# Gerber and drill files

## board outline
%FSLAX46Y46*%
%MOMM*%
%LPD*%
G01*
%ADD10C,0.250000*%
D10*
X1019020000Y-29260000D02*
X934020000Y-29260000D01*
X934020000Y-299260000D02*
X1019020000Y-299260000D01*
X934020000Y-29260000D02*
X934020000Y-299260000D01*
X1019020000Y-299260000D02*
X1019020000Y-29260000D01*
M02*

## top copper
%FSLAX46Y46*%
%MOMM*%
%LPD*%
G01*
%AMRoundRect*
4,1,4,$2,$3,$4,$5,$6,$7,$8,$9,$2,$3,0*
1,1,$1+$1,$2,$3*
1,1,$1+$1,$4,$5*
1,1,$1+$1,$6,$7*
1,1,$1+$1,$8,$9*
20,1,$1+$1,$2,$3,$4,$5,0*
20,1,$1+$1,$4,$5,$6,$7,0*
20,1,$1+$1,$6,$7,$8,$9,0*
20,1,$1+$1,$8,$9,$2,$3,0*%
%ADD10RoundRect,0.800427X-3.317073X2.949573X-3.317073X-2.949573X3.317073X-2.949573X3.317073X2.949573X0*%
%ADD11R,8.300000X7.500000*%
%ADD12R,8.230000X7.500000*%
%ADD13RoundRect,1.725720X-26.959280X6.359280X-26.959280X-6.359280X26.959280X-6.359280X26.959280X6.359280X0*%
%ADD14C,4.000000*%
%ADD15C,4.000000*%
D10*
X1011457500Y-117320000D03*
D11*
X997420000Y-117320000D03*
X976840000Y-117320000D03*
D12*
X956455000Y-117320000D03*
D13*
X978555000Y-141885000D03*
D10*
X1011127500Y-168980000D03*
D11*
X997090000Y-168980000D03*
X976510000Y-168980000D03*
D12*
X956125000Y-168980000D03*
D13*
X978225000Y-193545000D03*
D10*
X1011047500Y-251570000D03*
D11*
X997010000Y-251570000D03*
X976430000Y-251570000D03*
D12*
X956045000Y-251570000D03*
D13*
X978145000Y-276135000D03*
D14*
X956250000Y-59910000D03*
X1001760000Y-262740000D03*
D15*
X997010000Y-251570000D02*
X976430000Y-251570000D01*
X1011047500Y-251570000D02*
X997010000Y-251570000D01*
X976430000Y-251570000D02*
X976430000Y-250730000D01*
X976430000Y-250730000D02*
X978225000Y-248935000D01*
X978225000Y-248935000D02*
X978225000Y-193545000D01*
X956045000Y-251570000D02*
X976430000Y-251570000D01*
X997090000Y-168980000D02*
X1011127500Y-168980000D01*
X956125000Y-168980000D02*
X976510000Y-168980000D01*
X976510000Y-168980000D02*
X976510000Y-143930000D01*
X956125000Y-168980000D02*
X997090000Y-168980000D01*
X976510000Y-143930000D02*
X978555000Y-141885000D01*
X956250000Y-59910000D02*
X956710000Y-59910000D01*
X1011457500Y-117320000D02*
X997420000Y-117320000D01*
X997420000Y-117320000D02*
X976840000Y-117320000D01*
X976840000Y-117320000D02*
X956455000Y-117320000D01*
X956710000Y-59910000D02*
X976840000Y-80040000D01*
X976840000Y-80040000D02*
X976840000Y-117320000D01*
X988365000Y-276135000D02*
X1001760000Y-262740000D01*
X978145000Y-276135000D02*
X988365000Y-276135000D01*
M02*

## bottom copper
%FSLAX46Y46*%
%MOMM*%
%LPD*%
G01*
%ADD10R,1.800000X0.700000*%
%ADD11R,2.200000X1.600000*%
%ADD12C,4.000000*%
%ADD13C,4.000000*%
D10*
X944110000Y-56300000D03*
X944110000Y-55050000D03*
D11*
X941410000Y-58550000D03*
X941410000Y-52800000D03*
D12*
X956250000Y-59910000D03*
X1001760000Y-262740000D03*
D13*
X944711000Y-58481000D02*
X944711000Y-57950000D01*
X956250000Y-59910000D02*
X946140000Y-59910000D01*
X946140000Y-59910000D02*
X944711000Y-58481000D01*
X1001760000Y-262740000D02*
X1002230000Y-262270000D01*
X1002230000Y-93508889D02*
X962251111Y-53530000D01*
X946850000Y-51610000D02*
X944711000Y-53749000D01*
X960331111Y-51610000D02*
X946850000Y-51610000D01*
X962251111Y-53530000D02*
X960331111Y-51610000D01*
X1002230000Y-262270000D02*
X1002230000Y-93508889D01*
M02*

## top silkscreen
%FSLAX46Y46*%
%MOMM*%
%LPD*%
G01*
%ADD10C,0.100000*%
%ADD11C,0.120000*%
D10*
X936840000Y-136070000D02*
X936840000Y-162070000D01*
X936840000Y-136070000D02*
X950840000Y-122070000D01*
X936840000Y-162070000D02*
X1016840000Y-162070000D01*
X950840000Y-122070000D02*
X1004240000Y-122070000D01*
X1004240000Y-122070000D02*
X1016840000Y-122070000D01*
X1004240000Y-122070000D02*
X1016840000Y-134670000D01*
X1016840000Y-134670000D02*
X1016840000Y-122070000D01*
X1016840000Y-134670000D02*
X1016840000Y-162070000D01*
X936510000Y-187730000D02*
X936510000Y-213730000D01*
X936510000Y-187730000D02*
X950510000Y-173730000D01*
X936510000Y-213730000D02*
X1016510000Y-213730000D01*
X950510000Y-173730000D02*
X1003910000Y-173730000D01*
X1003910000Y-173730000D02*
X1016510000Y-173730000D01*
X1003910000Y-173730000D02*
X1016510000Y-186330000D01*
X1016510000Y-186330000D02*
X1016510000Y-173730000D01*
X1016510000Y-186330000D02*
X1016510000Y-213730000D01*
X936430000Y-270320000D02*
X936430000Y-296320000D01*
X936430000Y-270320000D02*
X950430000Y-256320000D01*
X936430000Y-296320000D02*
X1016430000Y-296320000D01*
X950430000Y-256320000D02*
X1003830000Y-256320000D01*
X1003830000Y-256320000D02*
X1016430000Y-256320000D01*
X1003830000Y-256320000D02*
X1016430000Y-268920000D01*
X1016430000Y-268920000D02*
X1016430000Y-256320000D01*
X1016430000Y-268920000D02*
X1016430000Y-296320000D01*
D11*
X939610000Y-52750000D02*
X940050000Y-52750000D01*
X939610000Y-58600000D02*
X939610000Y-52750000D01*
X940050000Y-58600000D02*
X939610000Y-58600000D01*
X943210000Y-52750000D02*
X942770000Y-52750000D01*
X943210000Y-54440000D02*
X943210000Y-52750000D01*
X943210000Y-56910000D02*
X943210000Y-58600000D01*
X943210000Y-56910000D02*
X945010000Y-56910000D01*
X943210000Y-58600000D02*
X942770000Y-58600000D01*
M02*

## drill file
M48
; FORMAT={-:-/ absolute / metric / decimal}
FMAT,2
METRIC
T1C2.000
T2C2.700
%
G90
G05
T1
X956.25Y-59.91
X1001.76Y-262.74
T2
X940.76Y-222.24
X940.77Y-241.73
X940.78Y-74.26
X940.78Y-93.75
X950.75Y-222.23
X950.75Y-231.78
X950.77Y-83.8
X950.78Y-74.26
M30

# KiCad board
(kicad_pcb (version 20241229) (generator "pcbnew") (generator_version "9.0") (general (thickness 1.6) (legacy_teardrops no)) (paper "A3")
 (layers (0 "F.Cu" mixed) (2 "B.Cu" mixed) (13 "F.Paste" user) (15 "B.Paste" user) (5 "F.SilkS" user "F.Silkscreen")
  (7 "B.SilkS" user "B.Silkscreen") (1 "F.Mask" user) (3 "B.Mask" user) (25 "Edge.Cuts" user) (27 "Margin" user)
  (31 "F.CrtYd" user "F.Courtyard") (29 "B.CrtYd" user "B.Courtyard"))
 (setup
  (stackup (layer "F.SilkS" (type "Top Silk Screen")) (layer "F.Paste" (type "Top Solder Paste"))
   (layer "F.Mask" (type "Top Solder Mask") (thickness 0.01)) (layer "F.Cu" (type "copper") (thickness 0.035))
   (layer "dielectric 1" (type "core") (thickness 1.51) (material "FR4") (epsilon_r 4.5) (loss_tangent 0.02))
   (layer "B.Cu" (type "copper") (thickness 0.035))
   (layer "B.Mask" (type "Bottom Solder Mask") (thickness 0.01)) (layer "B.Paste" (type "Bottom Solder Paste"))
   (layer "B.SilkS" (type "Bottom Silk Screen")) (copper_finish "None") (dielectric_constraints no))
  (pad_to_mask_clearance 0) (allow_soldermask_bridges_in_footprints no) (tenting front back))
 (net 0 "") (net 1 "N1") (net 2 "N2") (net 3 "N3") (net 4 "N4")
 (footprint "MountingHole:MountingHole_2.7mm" (layer "F.Cu") (at 940.78 93.75)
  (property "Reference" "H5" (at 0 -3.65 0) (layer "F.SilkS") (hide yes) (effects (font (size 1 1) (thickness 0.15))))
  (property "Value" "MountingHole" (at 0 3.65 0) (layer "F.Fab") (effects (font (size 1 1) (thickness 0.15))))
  (pad "" np_thru_hole circle (at 0 0) (size 2.7 2.7) (drill 2.7) (layers "*.Cu" "*.Mask")))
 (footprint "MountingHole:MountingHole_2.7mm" (layer "F.Cu") (at 940.76 222.24)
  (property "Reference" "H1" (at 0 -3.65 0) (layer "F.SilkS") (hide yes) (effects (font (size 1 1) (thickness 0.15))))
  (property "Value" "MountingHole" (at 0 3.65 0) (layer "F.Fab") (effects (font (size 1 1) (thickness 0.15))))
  (pad "" np_thru_hole circle (at 0 0) (size 2.7 2.7) (drill 2.7) (layers "*.Cu" "*.Mask")))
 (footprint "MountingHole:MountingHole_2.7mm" (layer "F.Cu") (at 950.75 231.78)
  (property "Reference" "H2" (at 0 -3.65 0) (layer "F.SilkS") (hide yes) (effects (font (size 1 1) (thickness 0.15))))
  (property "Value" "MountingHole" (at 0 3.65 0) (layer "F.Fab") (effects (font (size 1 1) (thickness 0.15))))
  (pad "" np_thru_hole circle (at 0 0) (size 2.7 2.7) (drill 2.7) (layers "*.Cu" "*.Mask")))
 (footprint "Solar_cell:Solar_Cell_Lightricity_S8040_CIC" (layer "F.Cu") (at 936.84 122.07 -90)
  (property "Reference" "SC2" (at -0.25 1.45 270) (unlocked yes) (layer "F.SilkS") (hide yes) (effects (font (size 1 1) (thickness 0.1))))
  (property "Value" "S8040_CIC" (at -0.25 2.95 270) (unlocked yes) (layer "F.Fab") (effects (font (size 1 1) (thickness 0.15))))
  (fp_line (start 14 0) (end 40 0) (stroke (width 0.1) (type default)) (layer "F.SilkS"))
  (fp_line (start 14 0) (end 0 -14) (stroke (width 0.1) (type default)) (layer "F.SilkS"))
  (fp_line (start 40 0) (end 40 -80) (stroke (width 0.1) (type default)) (layer "F.SilkS"))
  (fp_line (start 0 -14) (end 0 -67.4) (stroke (width 0.1) (type default)) (layer "F.SilkS"))
  (fp_line (start 0 -67.4) (end 0 -80) (stroke (width 0.1) (type default)) (layer "F.SilkS"))
  (fp_line (start 0 -67.4) (end 12.6 -80) (stroke (width 0.1) (type default)) (layer "F.SilkS"))
  (fp_line (start 12.6 -80) (end 0 -80) (stroke (width 0.1) (type default)) (layer "F.SilkS"))
  (fp_line (start 12.6 -80) (end 40 -80) (stroke (width 0.1) (type default)) (layer "F.SilkS"))
  (pad "1" smd roundrect (at -4.75 -74.6175 270) (size 7.5 8.235) (layers "F.Cu" "F.Mask" "F.Paste") (roundrect_rratio 0.1067235859)
   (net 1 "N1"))
  (pad "1" smd rect (at -4.75 -60.58 270) (size 7.5 8.3) (layers "F.Cu" "F.Mask" "F.Paste") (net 1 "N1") (thermal_bridge_angle 45))
  (pad "1" smd rect (at -4.75 -40 270) (size 7.5 8.3) (layers "F.Cu" "F.Mask" "F.Paste") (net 1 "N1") (thermal_bridge_angle 45))
  (pad "1" smd rect (at -4.75 -19.615 270) (size 7.5 8.23) (layers "F.Cu" "F.Mask" "F.Paste") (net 1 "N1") (thermal_bridge_angle 45))
  (pad "2" smd roundrect (at 19.815 -41.715 270) (size 16.17 57.37) (layers "F.Cu" "F.Mask" "F.Paste") (roundrect_rratio 0.1067235859)
   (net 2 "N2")))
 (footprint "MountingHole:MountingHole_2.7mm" (layer "F.Cu") (at 940.77 241.73)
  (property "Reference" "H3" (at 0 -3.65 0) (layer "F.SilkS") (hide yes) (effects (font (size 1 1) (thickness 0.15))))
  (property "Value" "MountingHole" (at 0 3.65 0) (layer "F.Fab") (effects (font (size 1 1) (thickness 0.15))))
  (pad "" np_thru_hole circle (at 0 0) (size 2.7 2.7) (drill 2.7) (layers "*.Cu" "*.Mask")))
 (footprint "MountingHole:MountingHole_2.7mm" (layer "F.Cu") (at 950.77 83.8)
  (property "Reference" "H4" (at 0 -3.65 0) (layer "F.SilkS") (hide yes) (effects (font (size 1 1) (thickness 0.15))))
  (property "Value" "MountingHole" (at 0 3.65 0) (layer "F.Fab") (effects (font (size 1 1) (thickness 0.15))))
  (pad "" np_thru_hole circle (at 0 0) (size 2.7 2.7) (drill 2.7) (layers "*.Cu" "*.Mask")))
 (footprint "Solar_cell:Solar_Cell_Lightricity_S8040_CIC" (layer "F.Cu") (at 936.51 173.73 -90)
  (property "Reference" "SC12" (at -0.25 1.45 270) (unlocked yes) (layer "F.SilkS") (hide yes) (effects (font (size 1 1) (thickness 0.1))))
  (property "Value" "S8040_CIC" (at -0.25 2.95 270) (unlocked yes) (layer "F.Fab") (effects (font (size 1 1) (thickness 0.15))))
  (fp_line (start 14 0) (end 40 0) (stroke (width 0.1) (type default)) (layer "F.SilkS"))
  (fp_line (start 14 0) (end 0 -14) (stroke (width 0.1) (type default)) (layer "F.SilkS"))
  (fp_line (start 40 0) (end 40 -80) (stroke (width 0.1) (type default)) (layer "F.SilkS"))
  (fp_line (start 0 -14) (end 0 -67.4) (stroke (width 0.1) (type default)) (layer "F.SilkS"))
  (fp_line (start 0 -67.4) (end 0 -80) (stroke (width 0.1) (type default)) (layer "F.SilkS"))
  (fp_line (start 0 -67.4) (end 12.6 -80) (stroke (width 0.1) (type default)) (layer "F.SilkS"))
  (fp_line (start 12.6 -80) (end 0 -80) (stroke (width 0.1) (type default)) (layer "F.SilkS"))
  (fp_line (start 12.6 -80) (end 40 -80) (stroke (width 0.1) (type default)) (layer "F.SilkS"))
  (pad "1" smd roundrect (at -4.75 -74.6175 270) (size 7.5 8.235) (layers "F.Cu" "F.Mask" "F.Paste") (roundrect_rratio 0.1067235859)
   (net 2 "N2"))
  (pad "1" smd rect (at -4.75 -60.58 270) (size 7.5 8.3) (layers "F.Cu" "F.Mask" "F.Paste") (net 2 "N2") (thermal_bridge_angle 45))
  (pad "1" smd rect (at -4.75 -40 270) (size 7.5 8.3) (layers "F.Cu" "F.Mask" "F.Paste") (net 2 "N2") (thermal_bridge_angle 45))
  (pad "1" smd rect (at -4.75 -19.615 270) (size 7.5 8.23) (layers "F.Cu" "F.Mask" "F.Paste") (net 2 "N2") (thermal_bridge_angle 45))
  (pad "2" smd roundrect (at 19.815 -41.715 270) (size 16.17 57.37) (layers "F.Cu" "F.Mask" "F.Paste") (roundrect_rratio 0.1067235859)
   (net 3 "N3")))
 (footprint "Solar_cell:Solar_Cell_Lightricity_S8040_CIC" (layer "F.Cu") (at 936.43 256.32 -90)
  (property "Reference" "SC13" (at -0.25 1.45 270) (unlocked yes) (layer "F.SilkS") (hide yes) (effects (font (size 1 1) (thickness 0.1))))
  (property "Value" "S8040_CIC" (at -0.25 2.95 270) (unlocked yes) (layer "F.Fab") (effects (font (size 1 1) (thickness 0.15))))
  (fp_line (start 14 0) (end 40 0) (stroke (width 0.1) (type default)) (layer "F.SilkS"))
  (fp_line (start 14 0) (end 0 -14) (stroke (width 0.1) (type default)) (layer "F.SilkS"))
  (fp_line (start 40 0) (end 40 -80) (stroke (width 0.1) (type default)) (layer "F.SilkS"))
  (fp_line (start 0 -14) (end 0 -67.4) (stroke (width 0.1) (type default)) (layer "F.SilkS"))
  (fp_line (start 0 -67.4) (end 0 -80) (stroke (width 0.1) (type default)) (layer "F.SilkS"))
  (fp_line (start 0 -67.4) (end 12.6 -80) (stroke (width 0.1) (type default)) (layer "F.SilkS"))
  (fp_line (start 12.6 -80) (end 0 -80) (stroke (width 0.1) (type default)) (layer "F.SilkS"))
  (fp_line (start 12.6 -80) (end 40 -80) (stroke (width 0.1) (type default)) (layer "F.SilkS"))
  (pad "1" smd roundrect (at -4.75 -74.6175 270) (size 7.5 8.235) (layers "F.Cu" "F.Mask" "F.Paste") (roundrect_rratio 0.1067235859)
   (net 3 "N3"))
  (pad "1" smd rect (at -4.75 -60.58 270) (size 7.5 8.3) (layers "F.Cu" "F.Mask" "F.Paste") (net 3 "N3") (thermal_bridge_angle 45))
  (pad "1" smd rect (at -4.75 -40 270) (size 7.5 8.3) (layers "F.Cu" "F.Mask" "F.Paste") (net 3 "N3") (thermal_bridge_angle 45))
  (pad "1" smd rect (at -4.75 -19.615 270) (size 7.5 8.23) (layers "F.Cu" "F.Mask" "F.Paste") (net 3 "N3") (thermal_bridge_angle 45))
  (pad "2" smd roundrect (at 19.815 -41.715 270) (size 16.17 57.37) (layers "F.Cu" "F.Mask" "F.Paste") (roundrect_rratio 0.1067235859)
   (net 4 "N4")))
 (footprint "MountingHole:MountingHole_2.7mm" (layer "F.Cu") (at 940.78 74.26)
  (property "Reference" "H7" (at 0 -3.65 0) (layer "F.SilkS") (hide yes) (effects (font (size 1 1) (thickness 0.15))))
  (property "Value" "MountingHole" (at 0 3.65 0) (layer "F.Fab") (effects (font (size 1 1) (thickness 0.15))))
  (pad "" np_thru_hole circle (at 0 0) (size 2.7 2.7) (drill 2.7) (layers "*.Cu" "*.Mask")))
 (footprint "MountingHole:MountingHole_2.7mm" (layer "F.Cu") (at 950.78 74.26)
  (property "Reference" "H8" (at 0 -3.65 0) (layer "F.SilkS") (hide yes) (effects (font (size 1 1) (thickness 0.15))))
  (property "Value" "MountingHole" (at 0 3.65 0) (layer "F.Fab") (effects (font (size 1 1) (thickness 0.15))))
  (pad "" np_thru_hole circle (at 0 0) (size 2.7 2.7) (drill 2.7) (layers "*.Cu" "*.Mask")))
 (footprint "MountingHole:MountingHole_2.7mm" (layer "F.Cu") (at 950.75 222.23)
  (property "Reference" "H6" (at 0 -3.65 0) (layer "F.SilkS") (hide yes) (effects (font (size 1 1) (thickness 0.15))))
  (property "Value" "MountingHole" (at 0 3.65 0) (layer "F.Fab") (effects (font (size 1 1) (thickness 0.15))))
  (pad "" np_thru_hole circle (at 0 0) (size 2.7 2.7) (drill 2.7) (layers "*.Cu" "*.Mask")))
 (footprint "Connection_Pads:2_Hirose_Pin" (layer "B.Cu") (at 950.51 49.855 90)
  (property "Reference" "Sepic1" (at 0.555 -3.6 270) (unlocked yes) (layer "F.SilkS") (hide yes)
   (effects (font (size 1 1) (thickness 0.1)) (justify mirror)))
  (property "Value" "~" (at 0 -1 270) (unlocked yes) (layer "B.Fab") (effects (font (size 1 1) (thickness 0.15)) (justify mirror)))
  (fp_line (start -2.895 -10.9) (end -2.895 -10.46) (stroke (width 0.12) (type solid)) (layer "F.SilkS"))
  (fp_line (start -8.745 -10.9) (end -2.895 -10.9) (stroke (width 0.12) (type solid)) (layer "F.SilkS"))
  (fp_line (start -8.745 -10.46) (end -8.745 -10.9) (stroke (width 0.12) (type solid)) (layer "F.SilkS"))
  (fp_line (start -2.895 -7.3) (end -2.895 -7.74) (stroke (width 0.12) (type solid)) (layer "F.SilkS"))
  (fp_line (start -4.585 -7.3) (end -2.895 -7.3) (stroke (width 0.12) (type solid)) (layer "F.SilkS"))
  (fp_line (start -7.055 -7.3) (end -8.745 -7.3) (stroke (width 0.12) (type solid)) (layer "F.SilkS"))
  (fp_line (start -7.055 -7.3) (end -7.055 -5.5) (stroke (width 0.12) (type solid)) (layer "F.SilkS"))
  (fp_line (start -8.745 -7.3) (end -8.745 -7.74) (stroke (width 0.12) (type solid)) (layer "F.SilkS"))
  (pad "1" smd rect (at -6.445 -6.4 90) (size 0.7 1.8) (layers "B.Cu" "B.Mask" "B.Paste") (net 1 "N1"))
  (pad "2" smd rect (at -5.195 -6.4 90) (size 0.7 1.8) (layers "B.Cu" "B.Mask" "B.Paste") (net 4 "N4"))
  (pad "MP" smd rect (at -8.695 -9.1 90) (size 1.6 2.2) (layers "B.Cu" "B.Mask" "B.Paste"))
  (pad "MP" smd rect (at -2.945 -9.1 90) (size 1.6 2.2) (layers "B.Cu" "B.Mask" "B.Paste")))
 (gr_line (start 1019.02 29.26) (end 934.02 29.26) (stroke (width 0.25) (type default)) (layer "Edge.Cuts"))
 (gr_line (start 934.02 299.26) (end 1019.02 299.26) (stroke (width 0.25) (type default)) (layer "Edge.Cuts"))
 (gr_line (start 934.02 29.26) (end 934.02 299.26) (stroke (width 0.25) (type default)) (layer "Edge.Cuts"))
 (gr_line (start 1019.02 299.26) (end 1019.02 29.26) (stroke (width 0.25) (type default)) (layer "Edge.Cuts"))
 (segment (start 997.01 251.57) (end 976.43 251.57) (width 4) (layer "F.Cu") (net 3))
 (segment (start 1011.0475 251.57) (end 997.01 251.57) (width 4) (layer "F.Cu") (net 3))
 (segment (start 976.43 251.57) (end 976.43 250.73) (width 4) (layer "F.Cu") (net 3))
 (segment (start 976.43 250.73) (end 978.225 248.935) (width 4) (layer "F.Cu") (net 3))
 (segment (start 978.225 248.935) (end 978.225 193.545) (width 4) (layer "F.Cu") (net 3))
 (segment (start 956.045 251.57) (end 976.43 251.57) (width 4) (layer "F.Cu") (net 3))
 (segment (start 997.09 168.98) (end 1011.1275 168.98) (width 4) (layer "F.Cu") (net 2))
 (segment (start 956.125 168.98) (end 976.51 168.98) (width 4) (layer "F.Cu") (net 2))
 (segment (start 976.51 168.98) (end 976.51 143.93) (width 4) (layer "F.Cu") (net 2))
 (segment (start 956.125 168.98) (end 997.09 168.98) (width 4) (layer "F.Cu") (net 2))
 (segment (start 976.51 143.93) (end 978.555 141.885) (width 4) (layer "F.Cu") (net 2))
 (segment (start 956.25 59.91) (end 956.71 59.91) (width 4) (layer "F.Cu") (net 1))
 (segment (start 1011.4575 117.32) (end 997.42 117.32) (width 4) (layer "F.Cu") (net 1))
 (segment (start 997.42 117.32) (end 976.84 117.32) (width 4) (layer "F.Cu") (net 1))
 (segment (start 976.84 117.32) (end 956.455 117.32) (width 4) (layer "F.Cu") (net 1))
 (segment (start 956.71 59.91) (end 976.84 80.04) (width 4) (layer "F.Cu") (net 1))
 (segment (start 976.84 80.04) (end 976.84 117.32) (width 4) (layer "F.Cu") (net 1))
 (via (at 956.25 59.91) (size 4) (drill 2) (layers "F.Cu" "B.Cu") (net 1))
 (segment (start 944.711 58.481) (end 944.711 57.95) (width 4) (layer "B.Cu") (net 1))
 (segment (start 956.25 59.91) (end 946.14 59.91) (width 4) (layer "B.Cu") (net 1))
 (segment (start 946.14 59.91) (end 944.711 58.481) (width 4) (layer "B.Cu") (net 1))
 (segment (start 988.365 276.135) (end 1001.76 262.74) (width 4) (layer "F.Cu") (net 4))
 (segment (start 978.145 276.135) (end 988.365 276.135) (width 4) (layer "F.Cu") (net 4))
 (via (at 1001.76 262.74) (size 4) (drill 2) (layers "F.Cu" "B.Cu") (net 4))
 (segment (start 1001.76 262.74) (end 1002.23 262.27) (width 4) (layer "B.Cu") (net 4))
 (segment (start 1002.23 93.508889) (end 962.251111 53.53) (width 4) (layer "B.Cu") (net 4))
 (segment (start 946.85 51.61) (end 944.711 53.749) (width 4) (layer "B.Cu") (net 4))
 (segment (start 960.331111 51.61) (end 946.85 51.61) (width 4) (layer "B.Cu") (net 4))
 (segment (start 962.251111 53.53) (end 960.331111 51.61) (width 4) (layer "B.Cu") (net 4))
 (segment (start 1002.23 262.27) (end 1002.23 93.508889) (width 4) (layer "B.Cu") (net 4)))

